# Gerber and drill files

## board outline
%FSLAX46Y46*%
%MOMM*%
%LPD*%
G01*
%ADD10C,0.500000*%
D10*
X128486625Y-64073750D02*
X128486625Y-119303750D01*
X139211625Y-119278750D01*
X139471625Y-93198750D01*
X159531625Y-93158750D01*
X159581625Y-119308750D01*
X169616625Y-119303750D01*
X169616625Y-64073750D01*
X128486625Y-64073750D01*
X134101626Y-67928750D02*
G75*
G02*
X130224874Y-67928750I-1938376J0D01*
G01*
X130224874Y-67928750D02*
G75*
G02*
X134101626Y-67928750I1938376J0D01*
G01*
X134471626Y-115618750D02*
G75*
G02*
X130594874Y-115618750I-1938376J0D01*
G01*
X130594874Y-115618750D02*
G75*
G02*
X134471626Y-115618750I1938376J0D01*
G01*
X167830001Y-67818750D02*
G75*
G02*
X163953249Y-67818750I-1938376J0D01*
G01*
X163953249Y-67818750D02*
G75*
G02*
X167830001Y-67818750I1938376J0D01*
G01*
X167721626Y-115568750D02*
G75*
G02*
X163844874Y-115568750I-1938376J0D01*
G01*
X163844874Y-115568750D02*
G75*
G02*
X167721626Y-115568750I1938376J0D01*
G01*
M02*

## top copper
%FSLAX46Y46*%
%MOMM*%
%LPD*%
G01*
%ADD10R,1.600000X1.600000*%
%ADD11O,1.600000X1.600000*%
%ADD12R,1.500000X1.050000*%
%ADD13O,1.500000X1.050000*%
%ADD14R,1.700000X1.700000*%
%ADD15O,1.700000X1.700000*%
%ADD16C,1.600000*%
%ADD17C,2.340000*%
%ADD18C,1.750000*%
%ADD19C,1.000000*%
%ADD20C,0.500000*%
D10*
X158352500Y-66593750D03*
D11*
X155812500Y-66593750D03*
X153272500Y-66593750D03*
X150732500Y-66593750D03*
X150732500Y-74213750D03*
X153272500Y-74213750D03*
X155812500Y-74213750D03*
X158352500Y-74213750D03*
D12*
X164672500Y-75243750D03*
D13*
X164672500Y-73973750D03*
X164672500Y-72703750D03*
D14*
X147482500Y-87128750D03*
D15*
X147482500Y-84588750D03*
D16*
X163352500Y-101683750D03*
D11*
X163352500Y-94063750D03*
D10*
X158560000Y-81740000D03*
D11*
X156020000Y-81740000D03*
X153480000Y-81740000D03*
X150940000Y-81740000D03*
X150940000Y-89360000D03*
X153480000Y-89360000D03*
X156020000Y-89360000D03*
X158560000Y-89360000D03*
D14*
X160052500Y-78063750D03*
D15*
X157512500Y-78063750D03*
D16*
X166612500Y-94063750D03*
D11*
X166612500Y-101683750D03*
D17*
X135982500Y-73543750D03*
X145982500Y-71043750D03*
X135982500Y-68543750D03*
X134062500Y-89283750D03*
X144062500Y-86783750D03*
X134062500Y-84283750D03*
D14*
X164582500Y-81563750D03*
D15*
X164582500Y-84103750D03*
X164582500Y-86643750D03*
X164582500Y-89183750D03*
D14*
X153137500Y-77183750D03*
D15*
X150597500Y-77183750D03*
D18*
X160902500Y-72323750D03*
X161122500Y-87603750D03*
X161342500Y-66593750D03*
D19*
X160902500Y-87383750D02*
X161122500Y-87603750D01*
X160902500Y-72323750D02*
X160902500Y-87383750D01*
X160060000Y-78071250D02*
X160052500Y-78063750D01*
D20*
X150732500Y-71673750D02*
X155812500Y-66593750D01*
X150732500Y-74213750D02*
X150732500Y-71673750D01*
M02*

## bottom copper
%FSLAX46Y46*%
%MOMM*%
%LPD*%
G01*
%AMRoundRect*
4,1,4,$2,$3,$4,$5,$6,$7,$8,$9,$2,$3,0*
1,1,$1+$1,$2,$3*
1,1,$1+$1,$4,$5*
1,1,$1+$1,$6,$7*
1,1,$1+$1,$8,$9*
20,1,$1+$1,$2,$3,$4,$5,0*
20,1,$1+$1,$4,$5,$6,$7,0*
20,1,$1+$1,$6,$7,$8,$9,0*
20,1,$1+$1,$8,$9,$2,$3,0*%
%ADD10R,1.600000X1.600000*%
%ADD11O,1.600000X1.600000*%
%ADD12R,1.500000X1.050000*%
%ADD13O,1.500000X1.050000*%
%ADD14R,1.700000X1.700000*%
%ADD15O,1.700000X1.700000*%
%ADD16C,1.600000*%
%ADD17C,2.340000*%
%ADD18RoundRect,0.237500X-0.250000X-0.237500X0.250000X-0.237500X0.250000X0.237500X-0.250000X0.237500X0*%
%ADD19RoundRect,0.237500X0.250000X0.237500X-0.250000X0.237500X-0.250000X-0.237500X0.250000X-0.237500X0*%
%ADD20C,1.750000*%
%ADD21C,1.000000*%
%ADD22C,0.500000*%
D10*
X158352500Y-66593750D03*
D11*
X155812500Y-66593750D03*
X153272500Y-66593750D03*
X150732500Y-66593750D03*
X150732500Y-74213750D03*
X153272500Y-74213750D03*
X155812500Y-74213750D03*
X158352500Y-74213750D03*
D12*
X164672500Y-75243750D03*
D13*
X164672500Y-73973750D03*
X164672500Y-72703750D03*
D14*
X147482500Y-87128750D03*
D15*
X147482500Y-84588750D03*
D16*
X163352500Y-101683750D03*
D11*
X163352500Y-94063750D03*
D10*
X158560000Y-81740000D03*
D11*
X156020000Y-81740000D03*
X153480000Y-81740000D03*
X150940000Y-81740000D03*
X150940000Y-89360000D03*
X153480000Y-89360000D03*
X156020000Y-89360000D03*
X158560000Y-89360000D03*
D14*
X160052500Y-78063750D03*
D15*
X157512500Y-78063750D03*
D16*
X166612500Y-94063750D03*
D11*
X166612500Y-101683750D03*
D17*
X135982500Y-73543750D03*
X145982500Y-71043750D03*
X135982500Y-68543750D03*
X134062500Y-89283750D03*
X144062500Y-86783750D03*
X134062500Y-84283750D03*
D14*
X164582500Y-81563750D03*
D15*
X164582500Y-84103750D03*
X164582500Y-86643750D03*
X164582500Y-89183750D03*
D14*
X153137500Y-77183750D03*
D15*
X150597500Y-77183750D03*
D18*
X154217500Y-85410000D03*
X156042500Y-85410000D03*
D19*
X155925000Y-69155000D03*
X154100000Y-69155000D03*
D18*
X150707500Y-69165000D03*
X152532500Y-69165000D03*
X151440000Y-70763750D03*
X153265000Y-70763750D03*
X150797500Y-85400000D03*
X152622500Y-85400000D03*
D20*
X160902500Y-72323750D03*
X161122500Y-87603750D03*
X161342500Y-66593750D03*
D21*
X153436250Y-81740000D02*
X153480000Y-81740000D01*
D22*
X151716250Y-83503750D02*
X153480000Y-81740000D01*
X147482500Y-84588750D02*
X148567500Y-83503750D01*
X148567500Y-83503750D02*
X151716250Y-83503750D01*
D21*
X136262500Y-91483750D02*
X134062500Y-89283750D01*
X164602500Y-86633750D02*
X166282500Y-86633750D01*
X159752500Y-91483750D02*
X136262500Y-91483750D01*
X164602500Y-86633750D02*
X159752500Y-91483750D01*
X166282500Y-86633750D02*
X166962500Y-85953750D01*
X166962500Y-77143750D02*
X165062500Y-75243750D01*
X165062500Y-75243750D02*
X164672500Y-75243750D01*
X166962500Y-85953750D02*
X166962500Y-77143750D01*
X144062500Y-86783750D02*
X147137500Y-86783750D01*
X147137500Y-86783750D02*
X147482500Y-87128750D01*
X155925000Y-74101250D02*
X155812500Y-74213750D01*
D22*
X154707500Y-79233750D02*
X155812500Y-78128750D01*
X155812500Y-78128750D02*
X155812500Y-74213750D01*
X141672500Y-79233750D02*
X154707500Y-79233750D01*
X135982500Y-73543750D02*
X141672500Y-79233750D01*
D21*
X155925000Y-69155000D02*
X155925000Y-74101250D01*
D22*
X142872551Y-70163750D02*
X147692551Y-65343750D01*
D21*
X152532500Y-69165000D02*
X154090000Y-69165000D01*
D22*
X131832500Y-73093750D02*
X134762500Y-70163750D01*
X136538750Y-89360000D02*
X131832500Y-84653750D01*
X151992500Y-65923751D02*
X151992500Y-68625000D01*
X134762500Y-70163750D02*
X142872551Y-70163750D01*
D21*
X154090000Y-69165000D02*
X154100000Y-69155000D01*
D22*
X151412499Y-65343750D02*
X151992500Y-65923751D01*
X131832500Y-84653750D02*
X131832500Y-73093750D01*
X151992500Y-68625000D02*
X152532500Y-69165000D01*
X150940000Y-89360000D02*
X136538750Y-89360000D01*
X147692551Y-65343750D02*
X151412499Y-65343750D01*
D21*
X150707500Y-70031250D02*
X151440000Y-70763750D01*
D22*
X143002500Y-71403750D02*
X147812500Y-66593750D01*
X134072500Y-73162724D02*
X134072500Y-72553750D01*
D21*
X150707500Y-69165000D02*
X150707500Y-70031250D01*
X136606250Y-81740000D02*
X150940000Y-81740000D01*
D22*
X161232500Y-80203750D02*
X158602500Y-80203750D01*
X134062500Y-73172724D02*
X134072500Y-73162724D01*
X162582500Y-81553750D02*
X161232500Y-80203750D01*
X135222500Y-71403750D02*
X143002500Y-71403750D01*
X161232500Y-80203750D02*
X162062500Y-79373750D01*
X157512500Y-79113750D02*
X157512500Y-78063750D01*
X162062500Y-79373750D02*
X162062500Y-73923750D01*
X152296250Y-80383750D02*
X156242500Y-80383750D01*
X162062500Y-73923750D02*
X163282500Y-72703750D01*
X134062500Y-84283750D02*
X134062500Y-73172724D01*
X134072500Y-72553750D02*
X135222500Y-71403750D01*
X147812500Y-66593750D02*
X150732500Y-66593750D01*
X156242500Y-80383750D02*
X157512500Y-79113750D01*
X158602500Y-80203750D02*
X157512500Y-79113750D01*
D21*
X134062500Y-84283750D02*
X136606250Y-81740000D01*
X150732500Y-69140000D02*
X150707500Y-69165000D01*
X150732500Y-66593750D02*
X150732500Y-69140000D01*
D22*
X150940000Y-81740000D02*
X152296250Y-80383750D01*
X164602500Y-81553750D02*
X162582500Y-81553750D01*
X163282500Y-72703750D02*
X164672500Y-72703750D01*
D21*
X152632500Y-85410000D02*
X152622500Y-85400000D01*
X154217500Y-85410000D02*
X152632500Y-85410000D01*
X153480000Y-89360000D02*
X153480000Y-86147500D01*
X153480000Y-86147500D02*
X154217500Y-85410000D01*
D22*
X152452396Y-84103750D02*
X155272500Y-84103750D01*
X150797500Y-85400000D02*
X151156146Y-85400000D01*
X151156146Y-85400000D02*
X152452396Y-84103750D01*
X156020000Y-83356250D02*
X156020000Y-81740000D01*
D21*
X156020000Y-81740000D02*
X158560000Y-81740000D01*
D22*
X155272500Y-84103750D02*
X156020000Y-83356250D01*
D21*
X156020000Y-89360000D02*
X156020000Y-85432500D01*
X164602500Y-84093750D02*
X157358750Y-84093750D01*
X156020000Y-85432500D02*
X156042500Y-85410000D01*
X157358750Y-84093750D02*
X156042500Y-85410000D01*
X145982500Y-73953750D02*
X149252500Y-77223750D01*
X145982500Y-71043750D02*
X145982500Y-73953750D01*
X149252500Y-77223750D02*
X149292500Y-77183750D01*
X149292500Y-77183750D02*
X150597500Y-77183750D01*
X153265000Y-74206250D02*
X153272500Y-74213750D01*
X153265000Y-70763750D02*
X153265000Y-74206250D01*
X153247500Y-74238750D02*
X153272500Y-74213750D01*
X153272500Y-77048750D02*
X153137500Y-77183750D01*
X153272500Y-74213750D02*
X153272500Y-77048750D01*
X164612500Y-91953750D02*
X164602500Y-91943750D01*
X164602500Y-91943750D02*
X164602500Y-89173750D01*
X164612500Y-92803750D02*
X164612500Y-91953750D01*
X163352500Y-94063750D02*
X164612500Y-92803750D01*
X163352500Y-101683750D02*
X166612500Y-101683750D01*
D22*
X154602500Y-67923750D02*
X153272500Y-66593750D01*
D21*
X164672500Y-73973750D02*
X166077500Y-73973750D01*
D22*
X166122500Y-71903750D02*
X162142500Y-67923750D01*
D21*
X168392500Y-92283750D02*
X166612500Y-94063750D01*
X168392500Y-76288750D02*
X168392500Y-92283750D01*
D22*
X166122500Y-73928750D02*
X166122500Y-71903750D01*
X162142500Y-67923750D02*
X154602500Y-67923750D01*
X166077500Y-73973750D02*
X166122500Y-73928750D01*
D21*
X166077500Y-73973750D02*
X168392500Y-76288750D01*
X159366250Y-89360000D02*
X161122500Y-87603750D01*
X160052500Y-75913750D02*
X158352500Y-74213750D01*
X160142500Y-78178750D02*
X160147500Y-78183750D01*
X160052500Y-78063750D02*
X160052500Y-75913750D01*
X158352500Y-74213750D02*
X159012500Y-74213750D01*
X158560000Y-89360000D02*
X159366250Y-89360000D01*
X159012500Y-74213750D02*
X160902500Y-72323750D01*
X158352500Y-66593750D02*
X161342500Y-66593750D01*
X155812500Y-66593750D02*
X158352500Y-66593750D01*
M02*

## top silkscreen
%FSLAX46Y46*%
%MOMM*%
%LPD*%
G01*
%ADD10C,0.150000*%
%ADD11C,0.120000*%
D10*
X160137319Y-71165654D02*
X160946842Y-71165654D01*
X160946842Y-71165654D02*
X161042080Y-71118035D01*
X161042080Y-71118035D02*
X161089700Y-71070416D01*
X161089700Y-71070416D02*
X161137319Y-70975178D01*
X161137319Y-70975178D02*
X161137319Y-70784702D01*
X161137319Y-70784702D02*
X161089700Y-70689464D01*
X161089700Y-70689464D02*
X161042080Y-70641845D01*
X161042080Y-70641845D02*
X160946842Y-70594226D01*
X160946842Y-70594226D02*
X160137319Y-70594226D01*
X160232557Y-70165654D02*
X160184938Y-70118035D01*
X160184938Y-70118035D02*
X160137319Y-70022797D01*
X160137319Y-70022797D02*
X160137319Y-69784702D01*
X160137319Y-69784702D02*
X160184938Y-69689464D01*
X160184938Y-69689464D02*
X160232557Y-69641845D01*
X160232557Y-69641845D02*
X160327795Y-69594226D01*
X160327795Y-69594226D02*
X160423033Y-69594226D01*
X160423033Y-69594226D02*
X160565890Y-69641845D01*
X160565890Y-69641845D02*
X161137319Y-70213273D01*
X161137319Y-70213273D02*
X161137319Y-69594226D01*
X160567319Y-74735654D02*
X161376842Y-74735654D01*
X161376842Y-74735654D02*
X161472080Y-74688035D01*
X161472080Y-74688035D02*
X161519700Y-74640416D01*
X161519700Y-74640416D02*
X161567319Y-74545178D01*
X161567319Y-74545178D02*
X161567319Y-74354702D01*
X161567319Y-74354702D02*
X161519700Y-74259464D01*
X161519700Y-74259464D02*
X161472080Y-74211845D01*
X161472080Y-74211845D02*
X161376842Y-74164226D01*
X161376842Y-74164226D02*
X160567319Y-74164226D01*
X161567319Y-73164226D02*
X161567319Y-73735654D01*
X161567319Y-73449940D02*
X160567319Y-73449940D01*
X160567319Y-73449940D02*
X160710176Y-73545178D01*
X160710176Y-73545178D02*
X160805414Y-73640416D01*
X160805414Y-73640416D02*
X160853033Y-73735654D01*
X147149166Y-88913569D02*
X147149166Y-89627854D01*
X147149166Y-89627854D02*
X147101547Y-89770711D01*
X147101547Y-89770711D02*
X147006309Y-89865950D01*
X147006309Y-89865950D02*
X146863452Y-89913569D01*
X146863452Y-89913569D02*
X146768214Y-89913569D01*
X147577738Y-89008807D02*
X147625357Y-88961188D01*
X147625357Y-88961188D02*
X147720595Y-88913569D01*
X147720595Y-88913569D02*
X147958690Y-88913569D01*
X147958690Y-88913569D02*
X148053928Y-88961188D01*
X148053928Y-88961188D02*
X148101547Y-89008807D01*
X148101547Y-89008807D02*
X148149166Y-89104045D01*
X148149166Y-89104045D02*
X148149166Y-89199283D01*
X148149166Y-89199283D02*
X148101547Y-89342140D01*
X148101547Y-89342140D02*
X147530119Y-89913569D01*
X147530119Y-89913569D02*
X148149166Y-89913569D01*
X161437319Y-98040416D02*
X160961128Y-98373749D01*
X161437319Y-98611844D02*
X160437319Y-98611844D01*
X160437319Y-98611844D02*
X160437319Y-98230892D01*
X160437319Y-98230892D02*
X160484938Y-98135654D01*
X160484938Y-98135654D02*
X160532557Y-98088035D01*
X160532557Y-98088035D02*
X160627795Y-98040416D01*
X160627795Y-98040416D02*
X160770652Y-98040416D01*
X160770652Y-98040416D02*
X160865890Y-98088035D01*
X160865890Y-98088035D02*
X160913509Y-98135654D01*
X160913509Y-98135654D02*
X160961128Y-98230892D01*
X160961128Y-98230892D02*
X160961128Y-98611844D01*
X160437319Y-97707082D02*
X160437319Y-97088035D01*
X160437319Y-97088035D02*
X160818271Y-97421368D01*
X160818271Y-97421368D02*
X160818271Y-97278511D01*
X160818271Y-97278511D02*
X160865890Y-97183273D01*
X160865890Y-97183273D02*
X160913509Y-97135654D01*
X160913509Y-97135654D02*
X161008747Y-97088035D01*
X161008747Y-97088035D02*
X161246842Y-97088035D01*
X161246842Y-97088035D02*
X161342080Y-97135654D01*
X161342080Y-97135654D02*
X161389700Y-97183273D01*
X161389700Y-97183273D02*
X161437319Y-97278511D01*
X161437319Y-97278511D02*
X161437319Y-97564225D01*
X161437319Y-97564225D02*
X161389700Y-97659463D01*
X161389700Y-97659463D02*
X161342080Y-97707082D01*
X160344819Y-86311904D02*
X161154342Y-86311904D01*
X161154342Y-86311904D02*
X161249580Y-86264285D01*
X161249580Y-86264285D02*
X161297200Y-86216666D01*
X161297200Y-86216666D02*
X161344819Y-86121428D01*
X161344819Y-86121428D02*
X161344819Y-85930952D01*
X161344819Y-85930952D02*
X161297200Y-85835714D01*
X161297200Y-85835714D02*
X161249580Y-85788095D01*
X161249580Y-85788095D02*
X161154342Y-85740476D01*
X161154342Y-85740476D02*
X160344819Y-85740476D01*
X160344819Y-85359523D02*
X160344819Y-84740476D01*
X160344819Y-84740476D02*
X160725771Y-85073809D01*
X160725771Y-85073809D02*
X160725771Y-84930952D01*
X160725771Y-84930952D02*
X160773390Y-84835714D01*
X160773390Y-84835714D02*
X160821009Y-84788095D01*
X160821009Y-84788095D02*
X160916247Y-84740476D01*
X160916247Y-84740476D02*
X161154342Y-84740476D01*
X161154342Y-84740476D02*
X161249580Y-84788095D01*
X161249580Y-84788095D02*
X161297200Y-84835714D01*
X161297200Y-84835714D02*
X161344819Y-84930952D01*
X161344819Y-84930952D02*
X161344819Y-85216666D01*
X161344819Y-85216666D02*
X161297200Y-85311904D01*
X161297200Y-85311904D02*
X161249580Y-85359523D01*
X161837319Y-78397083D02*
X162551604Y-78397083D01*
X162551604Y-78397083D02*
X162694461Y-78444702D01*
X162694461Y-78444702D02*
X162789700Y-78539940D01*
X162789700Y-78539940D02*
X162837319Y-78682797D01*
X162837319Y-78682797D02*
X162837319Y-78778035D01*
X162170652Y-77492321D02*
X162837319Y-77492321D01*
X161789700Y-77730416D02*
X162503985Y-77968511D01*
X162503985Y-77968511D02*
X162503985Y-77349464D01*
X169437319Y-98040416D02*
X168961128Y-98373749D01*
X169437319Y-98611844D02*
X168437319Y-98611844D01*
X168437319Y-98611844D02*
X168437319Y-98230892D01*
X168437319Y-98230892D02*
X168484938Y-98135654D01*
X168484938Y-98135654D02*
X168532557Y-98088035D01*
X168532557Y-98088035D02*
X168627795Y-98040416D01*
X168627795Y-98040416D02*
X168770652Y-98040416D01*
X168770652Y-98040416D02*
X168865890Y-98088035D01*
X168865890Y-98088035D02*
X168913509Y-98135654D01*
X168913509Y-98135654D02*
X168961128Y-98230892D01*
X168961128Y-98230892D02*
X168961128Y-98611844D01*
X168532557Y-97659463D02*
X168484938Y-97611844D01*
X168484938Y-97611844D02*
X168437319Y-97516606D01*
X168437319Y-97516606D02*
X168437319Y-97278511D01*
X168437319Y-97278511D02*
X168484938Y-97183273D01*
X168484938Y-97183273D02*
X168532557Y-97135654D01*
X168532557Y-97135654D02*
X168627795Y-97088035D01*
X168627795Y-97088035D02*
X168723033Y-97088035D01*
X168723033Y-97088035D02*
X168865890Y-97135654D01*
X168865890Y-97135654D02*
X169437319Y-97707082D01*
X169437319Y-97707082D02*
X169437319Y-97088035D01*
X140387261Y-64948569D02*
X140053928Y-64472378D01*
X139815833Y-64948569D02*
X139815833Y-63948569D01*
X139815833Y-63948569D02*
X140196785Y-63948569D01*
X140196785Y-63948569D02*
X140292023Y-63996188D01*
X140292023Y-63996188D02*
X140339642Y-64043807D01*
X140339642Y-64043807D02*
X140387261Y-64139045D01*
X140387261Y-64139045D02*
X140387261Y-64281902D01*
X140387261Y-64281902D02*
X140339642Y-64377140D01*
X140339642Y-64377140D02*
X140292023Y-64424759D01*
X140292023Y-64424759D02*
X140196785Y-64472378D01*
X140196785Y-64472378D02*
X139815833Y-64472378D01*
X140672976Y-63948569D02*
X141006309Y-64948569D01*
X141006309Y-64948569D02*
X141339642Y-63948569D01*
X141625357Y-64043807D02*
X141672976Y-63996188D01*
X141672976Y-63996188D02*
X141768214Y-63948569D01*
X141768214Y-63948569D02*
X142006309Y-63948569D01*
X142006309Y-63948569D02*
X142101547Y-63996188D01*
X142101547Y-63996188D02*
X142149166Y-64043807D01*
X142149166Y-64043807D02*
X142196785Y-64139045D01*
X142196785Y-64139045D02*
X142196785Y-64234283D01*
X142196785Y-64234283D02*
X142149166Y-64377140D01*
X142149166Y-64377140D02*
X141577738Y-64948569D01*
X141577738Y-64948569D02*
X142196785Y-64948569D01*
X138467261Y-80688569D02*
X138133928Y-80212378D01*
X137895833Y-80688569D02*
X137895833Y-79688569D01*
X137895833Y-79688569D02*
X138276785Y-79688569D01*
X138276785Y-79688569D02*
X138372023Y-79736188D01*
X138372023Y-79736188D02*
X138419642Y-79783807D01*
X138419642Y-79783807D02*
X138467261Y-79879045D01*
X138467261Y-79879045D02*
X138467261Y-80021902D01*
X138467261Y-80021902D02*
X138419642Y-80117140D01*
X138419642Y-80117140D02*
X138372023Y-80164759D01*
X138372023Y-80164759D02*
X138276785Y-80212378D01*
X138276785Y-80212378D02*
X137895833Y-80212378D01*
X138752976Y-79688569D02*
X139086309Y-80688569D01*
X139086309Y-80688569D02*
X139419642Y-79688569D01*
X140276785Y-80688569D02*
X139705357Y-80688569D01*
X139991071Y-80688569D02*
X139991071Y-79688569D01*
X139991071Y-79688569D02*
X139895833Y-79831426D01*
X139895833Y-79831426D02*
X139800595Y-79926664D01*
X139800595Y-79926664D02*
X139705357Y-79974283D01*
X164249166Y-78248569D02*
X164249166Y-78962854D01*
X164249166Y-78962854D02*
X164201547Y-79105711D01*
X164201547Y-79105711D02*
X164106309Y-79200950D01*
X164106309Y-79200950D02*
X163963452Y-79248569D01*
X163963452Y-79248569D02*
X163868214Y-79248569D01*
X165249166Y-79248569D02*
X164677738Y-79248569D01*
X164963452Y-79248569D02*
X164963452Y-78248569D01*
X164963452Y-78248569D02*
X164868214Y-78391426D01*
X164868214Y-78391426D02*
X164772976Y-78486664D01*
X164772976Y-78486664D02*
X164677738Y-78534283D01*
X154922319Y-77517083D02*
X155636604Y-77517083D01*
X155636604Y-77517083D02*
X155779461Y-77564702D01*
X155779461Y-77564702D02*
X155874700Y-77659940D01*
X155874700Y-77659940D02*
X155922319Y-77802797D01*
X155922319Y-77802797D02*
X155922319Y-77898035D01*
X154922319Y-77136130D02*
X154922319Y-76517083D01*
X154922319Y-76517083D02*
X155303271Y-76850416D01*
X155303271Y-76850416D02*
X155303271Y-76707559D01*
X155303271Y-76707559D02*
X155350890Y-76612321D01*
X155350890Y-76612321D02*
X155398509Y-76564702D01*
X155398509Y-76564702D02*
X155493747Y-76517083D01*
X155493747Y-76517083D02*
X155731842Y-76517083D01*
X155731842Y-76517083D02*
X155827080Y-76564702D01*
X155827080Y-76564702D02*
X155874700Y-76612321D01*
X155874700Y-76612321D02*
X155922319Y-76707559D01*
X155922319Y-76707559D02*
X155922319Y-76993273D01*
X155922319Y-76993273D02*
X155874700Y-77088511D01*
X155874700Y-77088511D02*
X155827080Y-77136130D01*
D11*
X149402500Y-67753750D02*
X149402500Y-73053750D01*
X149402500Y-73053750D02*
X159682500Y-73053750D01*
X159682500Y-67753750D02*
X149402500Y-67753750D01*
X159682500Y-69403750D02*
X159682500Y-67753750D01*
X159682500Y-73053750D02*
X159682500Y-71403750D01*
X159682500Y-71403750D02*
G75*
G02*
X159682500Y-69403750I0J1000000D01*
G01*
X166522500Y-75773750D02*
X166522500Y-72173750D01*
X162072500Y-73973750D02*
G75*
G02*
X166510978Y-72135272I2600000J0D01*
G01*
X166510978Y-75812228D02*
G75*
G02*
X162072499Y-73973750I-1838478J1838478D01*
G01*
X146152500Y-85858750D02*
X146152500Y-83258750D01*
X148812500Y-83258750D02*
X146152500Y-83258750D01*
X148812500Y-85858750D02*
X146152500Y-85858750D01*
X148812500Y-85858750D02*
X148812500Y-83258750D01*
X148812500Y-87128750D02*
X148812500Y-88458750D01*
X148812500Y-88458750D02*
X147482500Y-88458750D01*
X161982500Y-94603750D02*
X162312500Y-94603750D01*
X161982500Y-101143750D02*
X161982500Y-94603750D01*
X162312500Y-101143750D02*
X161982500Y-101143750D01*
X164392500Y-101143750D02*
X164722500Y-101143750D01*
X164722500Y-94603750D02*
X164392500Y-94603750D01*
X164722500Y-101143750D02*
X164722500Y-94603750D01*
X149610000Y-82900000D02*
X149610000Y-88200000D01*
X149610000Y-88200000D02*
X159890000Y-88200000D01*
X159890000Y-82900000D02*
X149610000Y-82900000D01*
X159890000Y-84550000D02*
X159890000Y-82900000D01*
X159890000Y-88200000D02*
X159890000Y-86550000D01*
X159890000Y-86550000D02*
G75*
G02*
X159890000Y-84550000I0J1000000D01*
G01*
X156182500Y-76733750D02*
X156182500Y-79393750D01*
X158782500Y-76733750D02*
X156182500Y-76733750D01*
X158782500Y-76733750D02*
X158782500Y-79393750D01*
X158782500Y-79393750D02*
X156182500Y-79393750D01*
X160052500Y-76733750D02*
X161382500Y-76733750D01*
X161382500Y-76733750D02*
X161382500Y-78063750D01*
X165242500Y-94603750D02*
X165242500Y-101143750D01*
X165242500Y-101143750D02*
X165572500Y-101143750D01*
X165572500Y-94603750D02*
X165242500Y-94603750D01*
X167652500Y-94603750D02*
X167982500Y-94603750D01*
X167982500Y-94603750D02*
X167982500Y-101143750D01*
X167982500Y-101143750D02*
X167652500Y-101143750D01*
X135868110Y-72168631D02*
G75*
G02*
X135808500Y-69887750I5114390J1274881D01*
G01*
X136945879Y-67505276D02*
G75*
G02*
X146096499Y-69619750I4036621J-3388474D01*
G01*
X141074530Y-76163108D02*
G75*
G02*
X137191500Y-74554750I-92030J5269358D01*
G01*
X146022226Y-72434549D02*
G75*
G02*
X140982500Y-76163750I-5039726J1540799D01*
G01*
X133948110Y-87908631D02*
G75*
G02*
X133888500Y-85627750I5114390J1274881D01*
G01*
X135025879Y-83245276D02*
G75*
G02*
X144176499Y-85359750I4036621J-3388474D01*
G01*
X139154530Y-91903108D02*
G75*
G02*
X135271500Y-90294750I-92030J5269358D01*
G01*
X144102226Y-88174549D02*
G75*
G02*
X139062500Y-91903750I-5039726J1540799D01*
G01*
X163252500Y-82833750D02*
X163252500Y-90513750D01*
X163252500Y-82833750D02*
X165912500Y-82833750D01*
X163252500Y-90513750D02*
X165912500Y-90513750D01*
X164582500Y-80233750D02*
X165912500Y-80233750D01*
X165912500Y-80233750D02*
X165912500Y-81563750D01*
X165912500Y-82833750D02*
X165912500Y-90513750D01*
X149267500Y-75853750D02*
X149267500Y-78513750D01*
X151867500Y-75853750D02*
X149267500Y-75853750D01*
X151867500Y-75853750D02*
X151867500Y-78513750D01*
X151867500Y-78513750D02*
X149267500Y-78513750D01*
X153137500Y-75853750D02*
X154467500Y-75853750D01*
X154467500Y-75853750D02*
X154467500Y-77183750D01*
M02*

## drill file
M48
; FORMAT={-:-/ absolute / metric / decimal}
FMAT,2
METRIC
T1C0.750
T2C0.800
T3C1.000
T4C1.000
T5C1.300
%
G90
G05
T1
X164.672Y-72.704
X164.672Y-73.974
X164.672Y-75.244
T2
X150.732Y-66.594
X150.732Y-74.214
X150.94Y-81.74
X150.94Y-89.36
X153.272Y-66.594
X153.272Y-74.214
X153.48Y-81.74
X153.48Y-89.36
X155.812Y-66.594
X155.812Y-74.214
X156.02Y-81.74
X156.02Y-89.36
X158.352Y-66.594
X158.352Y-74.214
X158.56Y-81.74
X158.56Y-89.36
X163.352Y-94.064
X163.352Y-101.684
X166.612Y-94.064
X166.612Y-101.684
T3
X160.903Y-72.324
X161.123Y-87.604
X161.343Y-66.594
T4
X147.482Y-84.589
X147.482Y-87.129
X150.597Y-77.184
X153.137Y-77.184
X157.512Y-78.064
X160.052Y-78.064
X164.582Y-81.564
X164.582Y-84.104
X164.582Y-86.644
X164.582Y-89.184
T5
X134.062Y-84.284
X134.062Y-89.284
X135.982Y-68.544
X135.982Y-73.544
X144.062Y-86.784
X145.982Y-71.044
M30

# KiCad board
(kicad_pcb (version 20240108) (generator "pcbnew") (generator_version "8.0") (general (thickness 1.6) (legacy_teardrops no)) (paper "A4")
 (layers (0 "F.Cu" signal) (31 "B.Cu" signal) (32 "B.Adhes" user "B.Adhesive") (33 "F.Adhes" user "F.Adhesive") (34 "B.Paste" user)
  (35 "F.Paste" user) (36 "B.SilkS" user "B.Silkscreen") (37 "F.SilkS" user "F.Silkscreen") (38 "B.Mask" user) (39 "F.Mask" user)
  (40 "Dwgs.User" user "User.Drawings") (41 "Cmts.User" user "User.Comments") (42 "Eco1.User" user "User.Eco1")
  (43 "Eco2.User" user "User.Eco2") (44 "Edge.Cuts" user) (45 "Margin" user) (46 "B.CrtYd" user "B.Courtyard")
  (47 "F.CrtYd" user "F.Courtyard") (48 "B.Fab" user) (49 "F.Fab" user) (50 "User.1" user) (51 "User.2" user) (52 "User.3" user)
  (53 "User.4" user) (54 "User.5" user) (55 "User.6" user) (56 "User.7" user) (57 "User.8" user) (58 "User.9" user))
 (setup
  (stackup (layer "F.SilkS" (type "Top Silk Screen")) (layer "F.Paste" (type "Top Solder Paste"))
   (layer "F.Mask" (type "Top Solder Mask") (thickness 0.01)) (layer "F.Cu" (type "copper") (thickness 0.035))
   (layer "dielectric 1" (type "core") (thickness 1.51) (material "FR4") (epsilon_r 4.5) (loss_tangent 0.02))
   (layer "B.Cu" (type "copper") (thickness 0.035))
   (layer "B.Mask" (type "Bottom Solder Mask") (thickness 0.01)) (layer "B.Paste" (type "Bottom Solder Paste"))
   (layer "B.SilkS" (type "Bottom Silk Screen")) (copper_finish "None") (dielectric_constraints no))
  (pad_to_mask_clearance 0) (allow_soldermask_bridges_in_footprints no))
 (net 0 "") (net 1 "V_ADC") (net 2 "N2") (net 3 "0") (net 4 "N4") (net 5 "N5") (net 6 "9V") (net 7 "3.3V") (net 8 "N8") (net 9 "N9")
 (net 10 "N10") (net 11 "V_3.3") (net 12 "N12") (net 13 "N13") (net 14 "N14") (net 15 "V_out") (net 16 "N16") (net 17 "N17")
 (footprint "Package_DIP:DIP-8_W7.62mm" (layer "F.Cu") (at 158.3525 66.59375 -90)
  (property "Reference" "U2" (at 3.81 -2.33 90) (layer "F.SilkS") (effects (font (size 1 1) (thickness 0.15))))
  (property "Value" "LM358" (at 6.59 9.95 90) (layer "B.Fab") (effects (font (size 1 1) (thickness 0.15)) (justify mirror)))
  (fp_line (start 1.16 8.95) (end 6.46 8.95) (stroke (width 0.12) (type solid)) (layer "F.SilkS"))
  (fp_line (start 6.46 8.95) (end 6.46 -1.33) (stroke (width 0.12) (type solid)) (layer "F.SilkS"))
  (fp_line (start 1.16 -1.33) (end 1.16 8.95) (stroke (width 0.12) (type solid)) (layer "F.SilkS"))
  (fp_line (start 2.81 -1.33) (end 1.16 -1.33) (stroke (width 0.12) (type solid)) (layer "F.SilkS"))
  (fp_line (start 6.46 -1.33) (end 4.81 -1.33) (stroke (width 0.12) (type solid)) (layer "F.SilkS"))
  (fp_arc (start 4.81 -1.33) (mid 3.81 -0.33) (end 2.81 -1.33) (stroke (width 0.12) (type solid)) (layer "F.SilkS"))
  (pad "1" thru_hole rect (at 0 0 270) (size 1.6 1.6) (drill 0.8) (layers "*.Cu" "*.Mask") (remove_unused_layers no) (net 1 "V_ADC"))
  (pad "2" thru_hole oval (at 0 2.54 270) (size 1.6 1.6) (drill 0.8) (layers "*.Cu" "*.Mask") (remove_unused_layers no) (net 1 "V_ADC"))
  (pad "3" thru_hole oval (at 0 5.08 270) (size 1.6 1.6) (drill 0.8) (layers "*.Cu" "*.Mask") (remove_unused_layers no) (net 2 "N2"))
  (pad "4" thru_hole oval (at 0 7.62 270) (size 1.6 1.6) (drill 0.8) (layers "*.Cu" "*.Mask") (remove_unused_layers no) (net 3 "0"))
  (pad "5" thru_hole oval (at 7.62 7.62 270) (size 1.6 1.6) (drill 0.8) (layers "*.Cu" "*.Mask") (remove_unused_layers no) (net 1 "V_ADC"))
  (pad "6" thru_hole oval (at 7.62 5.08 270) (size 1.6 1.6) (drill 0.8) (layers "*.Cu" "*.Mask") (remove_unused_layers no) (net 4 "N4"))
  (pad "7" thru_hole oval (at 7.62 2.54 270) (size 1.6 1.6) (drill 0.8) (layers "*.Cu" "*.Mask") (remove_unused_layers no) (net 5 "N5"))
  (pad "8" thru_hole oval (at 7.62 0 270) (size 1.6 1.6) (drill 0.8) (layers "*.Cu" "*.Mask") (remove_unused_layers no) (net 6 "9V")))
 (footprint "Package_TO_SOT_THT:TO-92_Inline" (layer "F.Cu") (at 164.6725 75.24375 90)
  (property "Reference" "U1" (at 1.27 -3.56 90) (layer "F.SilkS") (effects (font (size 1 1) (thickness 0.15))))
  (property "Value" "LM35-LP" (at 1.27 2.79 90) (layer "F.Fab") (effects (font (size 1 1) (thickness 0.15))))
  (fp_line (start -0.53 1.85) (end 3.07 1.85) (stroke (width 0.12) (type solid)) (layer "F.SilkS"))
  (fp_arc (start 1.27 -2.6) (mid 3.672087 -0.994977) (end 3.108478 1.838478) (stroke (width 0.12) (type solid)) (layer "F.SilkS"))
  (fp_arc (start -0.568478 1.838478) (mid -1.132087 -0.994977) (end 1.27 -2.6) (stroke (width 0.12) (type solid)) (layer "F.SilkS"))
  (pad "1" thru_hole rect (at 0 0 90) (size 1.05 1.5) (drill 0.75) (layers "*.Cu" "*.Mask") (remove_unused_layers no) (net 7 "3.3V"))
  (pad "2" thru_hole oval (at 1.27 0 90) (size 1.05 1.5) (drill 0.75) (layers "*.Cu" "*.Mask") (remove_unused_layers no) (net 2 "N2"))
  (pad "3" thru_hole oval (at 2.54 0 90) (size 1.05 1.5) (drill 0.75) (layers "*.Cu" "*.Mask") (remove_unused_layers no) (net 3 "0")))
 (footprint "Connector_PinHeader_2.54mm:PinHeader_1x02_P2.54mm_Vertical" (layer "F.Cu") (at 147.4825 87.12875 180)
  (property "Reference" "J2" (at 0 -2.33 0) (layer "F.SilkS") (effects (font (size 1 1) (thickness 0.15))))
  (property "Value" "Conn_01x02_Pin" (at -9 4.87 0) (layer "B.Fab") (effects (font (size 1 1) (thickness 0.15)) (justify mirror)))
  (fp_line (start 1.33 1.27) (end 1.33 3.87) (stroke (width 0.12) (type solid)) (layer "F.SilkS"))
  (fp_line (start -1.33 3.87) (end 1.33 3.87) (stroke (width 0.12) (type solid)) (layer "F.SilkS"))
  (fp_line (start -1.33 1.27) (end 1.33 1.27) (stroke (width 0.12) (type solid)) (layer "F.SilkS"))
  (fp_line (start -1.33 1.27) (end -1.33 3.87) (stroke (width 0.12) (type solid)) (layer "F.SilkS"))
  (fp_line (start -1.33 0) (end -1.33 -1.33) (stroke (width 0.12) (type solid)) (layer "F.SilkS"))
  (fp_line (start -1.33 -1.33) (end 0 -1.33) (stroke (width 0.12) (type solid)) (layer "F.SilkS"))
  (pad "1" thru_hole rect (at 0 0 180) (size 1.7 1.7) (drill 1) (layers "*.Cu" "*.Mask") (remove_unused_layers no) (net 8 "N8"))
  (pad "2" thru_hole oval (at 0 2.54 180) (size 1.7 1.7) (drill 1) (layers "*.Cu" "*.Mask") (remove_unused_layers no) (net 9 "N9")))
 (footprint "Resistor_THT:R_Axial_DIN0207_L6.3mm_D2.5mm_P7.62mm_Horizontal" (layer "F.Cu") (at 163.3525 101.68375 90)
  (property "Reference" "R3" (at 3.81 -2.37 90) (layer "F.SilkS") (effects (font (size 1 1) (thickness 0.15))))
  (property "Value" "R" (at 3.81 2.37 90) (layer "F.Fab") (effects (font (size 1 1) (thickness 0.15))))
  (fp_line (start 7.08 -1.37) (end 7.08 -1.04) (stroke (width 0.12) (type solid)) (layer "F.SilkS"))
  (fp_line (start 0.54 -1.37) (end 7.08 -1.37) (stroke (width 0.12) (type solid)) (layer "F.SilkS"))
  (fp_line (start 0.54 -1.04) (end 0.54 -1.37) (stroke (width 0.12) (type solid)) (layer "F.SilkS"))
  (fp_line (start 0.54 1.04) (end 0.54 1.37) (stroke (width 0.12) (type solid)) (layer "F.SilkS"))
  (fp_line (start 7.08 1.37) (end 7.08 1.04) (stroke (width 0.12) (type solid)) (layer "F.SilkS"))
  (fp_line (start 0.54 1.37) (end 7.08 1.37) (stroke (width 0.12) (type solid)) (layer "F.SilkS"))
  (pad "1" thru_hole circle (at 0 0 90) (size 1.6 1.6) (drill 0.8) (layers "*.Cu" "*.Mask") (remove_unused_layers no) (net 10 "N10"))
  (pad "2" thru_hole oval (at 7.62 0 90) (size 1.6 1.6) (drill 0.8) (layers "*.Cu" "*.Mask") (remove_unused_layers no) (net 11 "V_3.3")))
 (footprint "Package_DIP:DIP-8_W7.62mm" (layer "F.Cu") (at 158.56 81.74 -90)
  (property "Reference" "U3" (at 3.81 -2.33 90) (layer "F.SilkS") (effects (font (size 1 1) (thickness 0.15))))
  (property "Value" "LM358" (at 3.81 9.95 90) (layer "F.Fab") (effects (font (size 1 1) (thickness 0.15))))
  (fp_line (start 1.16 8.95) (end 6.46 8.95) (stroke (width 0.12) (type solid)) (layer "F.SilkS"))
  (fp_line (start 6.46 8.95) (end 6.46 -1.33) (stroke (width 0.12) (type solid)) (layer "F.SilkS"))
  (fp_line (start 1.16 -1.33) (end 1.16 8.95) (stroke (width 0.12) (type solid)) (layer "F.SilkS"))
  (fp_line (start 2.81 -1.33) (end 1.16 -1.33) (stroke (width 0.12) (type solid)) (layer "F.SilkS"))
  (fp_line (start 6.46 -1.33) (end 4.81 -1.33) (stroke (width 0.12) (type solid)) (layer "F.SilkS"))
  (fp_arc (start 4.81 -1.33) (mid 3.81 -0.33) (end 2.81 -1.33) (stroke (width 0.12) (type solid)) (layer "F.SilkS"))
  (pad "1" thru_hole rect (at 0 0 270) (size 1.6 1.6) (drill 0.8) (layers "*.Cu" "*.Mask") (remove_unused_layers no) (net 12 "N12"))
  (pad "2" thru_hole oval (at 0 2.54 270) (size 1.6 1.6) (drill 0.8) (layers "*.Cu" "*.Mask") (remove_unused_layers no) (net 12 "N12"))
  (pad "3" thru_hole oval (at 0 5.08 270) (size 1.6 1.6) (drill 0.8) (layers "*.Cu" "*.Mask") (remove_unused_layers no) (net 9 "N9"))
  (pad "4" thru_hole oval (at 0 7.62 270) (size 1.6 1.6) (drill 0.8) (layers "*.Cu" "*.Mask") (remove_unused_layers no) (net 3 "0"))
  (pad "5" thru_hole oval (at 7.62 7.62 270) (size 1.6 1.6) (drill 0.8) (layers "*.Cu" "*.Mask") (remove_unused_layers no) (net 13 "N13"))
  (pad "6" thru_hole oval (at 7.62 5.08 270) (size 1.6 1.6) (drill 0.8) (layers "*.Cu" "*.Mask") (remove_unused_layers no) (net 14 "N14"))
  (pad "7" thru_hole oval (at 7.62 2.54 270) (size 1.6 1.6) (drill 0.8) (layers "*.Cu" "*.Mask") (remove_unused_layers no) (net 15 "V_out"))
  (pad "8" thru_hole oval (at 7.62 0 270) (size 1.6 1.6) (drill 0.8) (layers "*.Cu" "*.Mask") (remove_unused_layers no) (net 6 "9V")))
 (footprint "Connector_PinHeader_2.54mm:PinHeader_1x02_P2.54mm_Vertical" (layer "F.Cu") (at 160.0525 78.06375 -90)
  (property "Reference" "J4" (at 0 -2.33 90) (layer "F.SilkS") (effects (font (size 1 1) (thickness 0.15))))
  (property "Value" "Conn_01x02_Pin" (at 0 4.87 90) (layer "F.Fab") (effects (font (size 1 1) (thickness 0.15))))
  (fp_line (start -1.33 3.87) (end 1.33 3.87) (stroke (width 0.12) (type solid)) (layer "F.SilkS"))
  (fp_line (start -1.33 1.27) (end -1.33 3.87) (stroke (width 0.12) (type solid)) (layer "F.SilkS"))
  (fp_line (start -1.33 1.27) (end 1.33 1.27) (stroke (width 0.12) (type solid)) (layer "F.SilkS"))
  (fp_line (start 1.33 1.27) (end 1.33 3.87) (stroke (width 0.12) (type solid)) (layer "F.SilkS"))
  (fp_line (start -1.33 0) (end -1.33 -1.33) (stroke (width 0.12) (type solid)) (layer "F.SilkS"))
  (fp_line (start -1.33 -1.33) (end 0 -1.33) (stroke (width 0.12) (type solid)) (layer "F.SilkS"))
  (pad "1" thru_hole rect (at 0 0 270) (size 1.7 1.7) (drill 1) (layers "*.Cu" "*.Mask") (remove_unused_layers no) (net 6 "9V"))
  (pad "2" thru_hole oval (at 0 2.54 270) (size 1.7 1.7) (drill 1) (layers "*.Cu" "*.Mask") (remove_unused_layers no) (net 3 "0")))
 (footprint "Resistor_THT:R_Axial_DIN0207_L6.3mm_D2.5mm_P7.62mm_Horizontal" (layer "F.Cu") (at 166.6125 94.06375 -90)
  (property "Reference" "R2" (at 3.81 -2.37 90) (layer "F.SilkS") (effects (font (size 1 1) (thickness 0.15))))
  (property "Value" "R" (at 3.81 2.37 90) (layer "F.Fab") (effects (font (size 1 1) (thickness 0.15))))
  (fp_line (start 0.54 1.37) (end 7.08 1.37) (stroke (width 0.12) (type solid)) (layer "F.SilkS"))
  (fp_line (start 7.08 1.37) (end 7.08 1.04) (stroke (width 0.12) (type solid)) (layer "F.SilkS"))
  (fp_line (start 0.54 1.04) (end 0.54 1.37) (stroke (width 0.12) (type solid)) (layer "F.SilkS"))
  (fp_line (start 0.54 -1.04) (end 0.54 -1.37) (stroke (width 0.12) (type solid)) (layer "F.SilkS"))
  (fp_line (start 0.54 -1.37) (end 7.08 -1.37) (stroke (width 0.12) (type solid)) (layer "F.SilkS"))
  (fp_line (start 7.08 -1.37) (end 7.08 -1.04) (stroke (width 0.12) (type solid)) (layer "F.SilkS"))
  (pad "1" thru_hole circle (at 0 0 270) (size 1.6 1.6) (drill 0.8) (layers "*.Cu" "*.Mask") (remove_unused_layers no) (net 2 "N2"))
  (pad "2" thru_hole oval (at 7.62 0 270) (size 1.6 1.6) (drill 0.8) (layers "*.Cu" "*.Mask") (remove_unused_layers no) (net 10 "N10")))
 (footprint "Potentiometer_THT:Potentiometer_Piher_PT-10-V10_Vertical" (layer "F.Cu") (at 135.9825 73.54375)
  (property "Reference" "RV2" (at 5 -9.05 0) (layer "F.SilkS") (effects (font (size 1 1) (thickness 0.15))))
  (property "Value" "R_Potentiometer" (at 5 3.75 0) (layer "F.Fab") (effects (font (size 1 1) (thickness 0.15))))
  (fp_arc (start -0.11439 -1.375119) (mid -0.269093 -2.512295) (end -0.174 -3.656) (stroke (width 0.12) (type solid)) (layer "F.SilkS"))
  (fp_arc (start 0.963379 -6.038474) (mid 6.186565 -7.784991) (end 10.114 -3.924) (stroke (width 0.12) (type solid)) (layer "F.SilkS"))
  (fp_arc (start 5.09203 2.619358) (mid 2.983245 2.219015) (end 1.209 1.011) (stroke (width 0.12) (type solid)) (layer "F.SilkS"))
  (fp_arc (start 10.039726 -1.109201) (mid 8.134716 1.586326) (end 5 2.62) (stroke (width 0.12) (type solid)) (layer "F.SilkS"))
  (pad "1" thru_hole circle (at 0 0) (size 2.34 2.34) (drill 1.3) (layers "*.Cu" "*.Mask") (remove_unused_layers no) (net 5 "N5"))
  (pad "2" thru_hole circle (at 10 -2.5) (size 2.34 2.34) (drill 1.3) (layers "*.Cu" "*.Mask") (remove_unused_layers no) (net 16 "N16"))
  (pad "3" thru_hole circle (at 0 -5) (size 2.34 2.34) (drill 1.3) (layers "*.Cu" "*.Mask") (remove_unused_layers no) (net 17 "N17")))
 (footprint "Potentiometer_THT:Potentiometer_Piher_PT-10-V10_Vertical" (layer "F.Cu") (at 134.0625 89.28375)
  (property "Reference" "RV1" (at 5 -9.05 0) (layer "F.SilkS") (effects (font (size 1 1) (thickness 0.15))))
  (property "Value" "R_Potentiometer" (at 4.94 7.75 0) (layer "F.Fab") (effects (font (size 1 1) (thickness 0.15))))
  (fp_arc (start -0.11439 -1.375119) (mid -0.269093 -2.512295) (end -0.174 -3.656) (stroke (width 0.12) (type solid)) (layer "F.SilkS"))
  (fp_arc (start 0.963379 -6.038474) (mid 6.186565 -7.784991) (end 10.114 -3.924) (stroke (width 0.12) (type solid)) (layer "F.SilkS"))
  (fp_arc (start 5.09203 2.619358) (mid 2.983245 2.219015) (end 1.209 1.011) (stroke (width 0.12) (type solid)) (layer "F.SilkS"))
  (fp_arc (start 10.039726 -1.109201) (mid 8.134716 1.586326) (end 5 2.62) (stroke (width 0.12) (type solid)) (layer "F.SilkS"))
  (pad "1" thru_hole circle (at 0 0) (size 2.34 2.34) (drill 1.3) (layers "*.Cu" "*.Mask") (remove_unused_layers no) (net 7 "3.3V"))
  (pad "2" thru_hole circle (at 10 -2.5) (size 2.34 2.34) (drill 1.3) (layers "*.Cu" "*.Mask") (remove_unused_layers no) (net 8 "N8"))
  (pad "3" thru_hole circle (at 0 -5) (size 2.34 2.34) (drill 1.3) (layers "*.Cu" "*.Mask") (remove_unused_layers no) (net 3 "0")))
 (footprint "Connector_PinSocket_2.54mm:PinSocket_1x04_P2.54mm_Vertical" (layer "F.Cu") (at 164.5825 81.56375)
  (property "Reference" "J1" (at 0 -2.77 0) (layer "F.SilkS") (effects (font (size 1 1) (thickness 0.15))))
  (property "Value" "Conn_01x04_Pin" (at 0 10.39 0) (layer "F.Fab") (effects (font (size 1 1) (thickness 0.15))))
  (fp_line (start -1.33 1.27) (end -1.33 8.95) (stroke (width 0.12) (type solid)) (layer "F.SilkS"))
  (fp_line (start -1.33 1.27) (end 1.33 1.27) (stroke (width 0.12) (type solid)) (layer "F.SilkS"))
  (fp_line (start -1.33 8.95) (end 1.33 8.95) (stroke (width 0.12) (type solid)) (layer "F.SilkS"))
  (fp_line (start 0 -1.33) (end 1.33 -1.33) (stroke (width 0.12) (type solid)) (layer "F.SilkS"))
  (fp_line (start 1.33 -1.33) (end 1.33 0) (stroke (width 0.12) (type solid)) (layer "F.SilkS"))
  (fp_line (start 1.33 1.27) (end 1.33 8.95) (stroke (width 0.12) (type solid)) (layer "F.SilkS"))
  (pad "1" thru_hole rect (at 0 0) (size 1.7 1.7) (drill 1) (layers "*.Cu" "*.Mask") (remove_unused_layers no) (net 3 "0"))
  (pad "2" thru_hole oval (at 0 2.54) (size 1.7 1.7) (drill 1) (layers "*.Cu" "*.Mask") (remove_unused_layers no) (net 15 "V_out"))
  (pad "3" thru_hole oval (at 0 5.08) (size 1.7 1.7) (drill 1) (layers "*.Cu" "*.Mask") (remove_unused_layers no) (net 7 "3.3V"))
  (pad "4" thru_hole oval (at 0 7.62) (size 1.7 1.7) (drill 1) (layers "*.Cu" "*.Mask") (remove_unused_layers no) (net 11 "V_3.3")))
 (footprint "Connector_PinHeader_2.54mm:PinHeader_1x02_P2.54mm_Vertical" (layer "F.Cu") (at 153.1375 77.18375 -90)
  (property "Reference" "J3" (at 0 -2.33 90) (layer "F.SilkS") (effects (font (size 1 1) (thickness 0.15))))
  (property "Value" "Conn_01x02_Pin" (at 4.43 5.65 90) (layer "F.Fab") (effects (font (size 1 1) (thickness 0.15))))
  (fp_line (start -1.33 3.87) (end 1.33 3.87) (stroke (width 0.12) (type solid)) (layer "F.SilkS"))
  (fp_line (start -1.33 1.27) (end -1.33 3.87) (stroke (width 0.12) (type solid)) (layer "F.SilkS"))
  (fp_line (start -1.33 1.27) (end 1.33 1.27) (stroke (width 0.12) (type solid)) (layer "F.SilkS"))
  (fp_line (start 1.33 1.27) (end 1.33 3.87) (stroke (width 0.12) (type solid)) (layer "F.SilkS"))
  (fp_line (start -1.33 0) (end -1.33 -1.33) (stroke (width 0.12) (type solid)) (layer "F.SilkS"))
  (fp_line (start -1.33 -1.33) (end 0 -1.33) (stroke (width 0.12) (type solid)) (layer "F.SilkS"))
  (pad "1" thru_hole rect (at 0 0 270) (size 1.7 1.7) (drill 1) (layers "*.Cu" "*.Mask") (remove_unused_layers no) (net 4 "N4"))
  (pad "2" thru_hole oval (at 0 2.54 270) (size 1.7 1.7) (drill 1) (layers "*.Cu" "*.Mask") (remove_unused_layers no) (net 16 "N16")))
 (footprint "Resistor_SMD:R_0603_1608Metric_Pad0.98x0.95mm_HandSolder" (layer "B.Cu") (at 155.13 85.41)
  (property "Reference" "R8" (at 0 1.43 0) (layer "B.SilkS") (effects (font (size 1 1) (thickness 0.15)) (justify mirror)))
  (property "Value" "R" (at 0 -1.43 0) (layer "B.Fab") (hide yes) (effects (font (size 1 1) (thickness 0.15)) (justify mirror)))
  (pad "1" smd roundrect (at -0.9125 0) (size 0.975 0.95) (layers "B.Cu" "B.Paste" "B.Mask") (roundrect_rratio 0.25) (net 14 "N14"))
  (pad "2" smd roundrect (at 0.9125 0) (size 0.975 0.95) (layers "B.Cu" "B.Paste" "B.Mask") (roundrect_rratio 0.25) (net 15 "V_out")))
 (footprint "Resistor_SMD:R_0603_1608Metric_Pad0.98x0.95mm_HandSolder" (layer "B.Cu") (at 155.0125 69.155 180)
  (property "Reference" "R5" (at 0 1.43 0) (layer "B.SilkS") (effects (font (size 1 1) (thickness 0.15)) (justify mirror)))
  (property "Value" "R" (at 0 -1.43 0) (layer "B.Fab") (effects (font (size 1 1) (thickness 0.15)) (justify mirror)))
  (pad "1" smd roundrect (at -0.9125 0 180) (size 0.975 0.95) (layers "B.Cu" "B.Paste" "B.Mask") (roundrect_rratio 0.25) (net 5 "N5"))
  (pad "2" smd roundrect (at 0.9125 0 180) (size 0.975 0.95) (layers "B.Cu" "B.Paste" "B.Mask") (roundrect_rratio 0.25) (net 13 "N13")))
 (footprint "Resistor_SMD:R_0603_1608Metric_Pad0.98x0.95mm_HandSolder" (layer "B.Cu") (at 151.62 69.165)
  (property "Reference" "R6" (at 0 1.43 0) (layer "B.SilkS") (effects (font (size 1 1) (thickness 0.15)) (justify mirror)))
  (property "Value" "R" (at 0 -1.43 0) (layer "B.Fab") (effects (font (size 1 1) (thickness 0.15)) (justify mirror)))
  (pad "1" smd roundrect (at -0.9125 0) (size 0.975 0.95) (layers "B.Cu" "B.Paste" "B.Mask") (roundrect_rratio 0.25) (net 3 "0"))
  (pad "2" smd roundrect (at 0.9125 0) (size 0.975 0.95) (layers "B.Cu" "B.Paste" "B.Mask") (roundrect_rratio 0.25) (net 13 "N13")))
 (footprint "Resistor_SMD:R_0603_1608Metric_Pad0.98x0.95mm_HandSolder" (layer "B.Cu") (at 152.3525 70.76375)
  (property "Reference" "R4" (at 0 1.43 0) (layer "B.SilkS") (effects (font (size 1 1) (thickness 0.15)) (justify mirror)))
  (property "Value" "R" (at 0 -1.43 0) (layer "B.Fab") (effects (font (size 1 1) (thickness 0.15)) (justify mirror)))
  (pad "1" smd roundrect (at -0.9125 0) (size 0.975 0.95) (layers "B.Cu" "B.Paste" "B.Mask") (roundrect_rratio 0.25) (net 3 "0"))
  (pad "2" smd roundrect (at 0.9125 0) (size 0.975 0.95) (layers "B.Cu" "B.Paste" "B.Mask") (roundrect_rratio 0.25) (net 4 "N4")))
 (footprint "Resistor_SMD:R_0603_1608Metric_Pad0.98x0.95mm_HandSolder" (layer "B.Cu") (at 151.71 85.4)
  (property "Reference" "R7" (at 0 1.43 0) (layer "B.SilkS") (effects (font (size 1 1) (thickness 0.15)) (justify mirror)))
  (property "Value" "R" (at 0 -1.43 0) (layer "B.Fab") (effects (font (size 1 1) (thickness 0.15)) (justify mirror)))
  (pad "1" smd roundrect (at -0.9125 0) (size 0.975 0.95) (layers "B.Cu" "B.Paste" "B.Mask") (roundrect_rratio 0.25) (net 12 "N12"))
  (pad "2" smd roundrect (at 0.9125 0) (size 0.975 0.95) (layers "B.Cu" "B.Paste" "B.Mask") (roundrect_rratio 0.25) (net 14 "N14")))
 (gr_poly
  (pts (xy 128.486625 64.07375) (xy 128.486625 119.30375) (xy 139.211625 119.27875) (xy 139.471625 93.19875) (xy 159.531625 93.15875)
   (xy 159.581625 119.30875) (xy 169.616625 119.30375) (xy 169.616625 64.07375))
  (stroke (width 0.5) (type solid)) (fill none) (layer "Edge.Cuts"))
 (gr_circle (center 132.16325 67.92875) (end 134.101626 67.92875) (stroke (width 0.5) (type default)) (fill none) (layer "Edge.Cuts"))
 (gr_circle (center 132.53325 115.61875) (end 134.471626 115.61875) (stroke (width 0.5) (type default)) (fill none) (layer "Edge.Cuts"))
 (gr_circle (center 165.891625 67.81875) (end 167.830001 67.81875) (stroke (width 0.5) (type default)) (fill none) (layer "Edge.Cuts"))
 (gr_circle (center 165.78325 115.56875) (end 167.721626 115.56875) (stroke (width 0.5) (type default)) (fill none) (layer "Edge.Cuts"))
 (segment (start 153.43625 81.74) (end 153.48 81.74) (width 1) (layer "B.Cu") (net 9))
 (segment (start 151.71625 83.50375) (end 153.48 81.74) (width 0.5) (layer "B.Cu") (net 9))
 (segment (start 147.4825 84.58875) (end 148.5675 83.50375) (width 0.5) (layer "B.Cu") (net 9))
 (segment (start 148.5675 83.50375) (end 151.71625 83.50375) (width 0.5) (layer "B.Cu") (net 9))
 (segment (start 136.2625 91.48375) (end 134.0625 89.28375) (width 1) (layer "B.Cu") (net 7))
 (segment (start 164.6025 86.63375) (end 166.2825 86.63375) (width 1) (layer "B.Cu") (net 7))
 (segment (start 159.7525 91.48375) (end 136.2625 91.48375) (width 1) (layer "B.Cu") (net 7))
 (segment (start 164.6025 86.63375) (end 159.7525 91.48375) (width 1) (layer "B.Cu") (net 7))
 (segment (start 166.2825 86.63375) (end 166.9625 85.95375) (width 1) (layer "B.Cu") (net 7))
 (segment (start 166.9625 77.14375) (end 165.0625 75.24375) (width 1) (layer "B.Cu") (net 7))
 (segment (start 165.0625 75.24375) (end 164.6725 75.24375) (width 1) (layer "B.Cu") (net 7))
 (segment (start 166.9625 85.95375) (end 166.9625 77.14375) (width 1) (layer "B.Cu") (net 7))
 (segment (start 144.0625 86.78375) (end 147.1375 86.78375) (width 1) (layer "B.Cu") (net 8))
 (segment (start 147.1375 86.78375) (end 147.4825 87.12875) (width 1) (layer "B.Cu") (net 8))
 (segment (start 155.925 74.10125) (end 155.8125 74.21375) (width 1) (layer "B.Cu") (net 5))
 (segment (start 154.7075 79.23375) (end 155.8125 78.12875) (width 0.5) (layer "B.Cu") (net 5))
 (segment (start 155.8125 78.12875) (end 155.8125 74.21375) (width 0.5) (layer "B.Cu") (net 5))
 (segment (start 141.6725 79.23375) (end 154.7075 79.23375) (width 0.5) (layer "B.Cu") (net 5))
 (segment (start 135.9825 73.54375) (end 141.6725 79.23375) (width 0.5) (layer "B.Cu") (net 5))
 (segment (start 155.925 69.155) (end 155.925 74.10125) (width 1) (layer "B.Cu") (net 5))
 (segment (start 142.872551 70.16375) (end 147.692551 65.34375) (width 0.5) (layer "B.Cu") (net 13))
 (segment (start 152.5325 69.165) (end 154.09 69.165) (width 1) (layer "B.Cu") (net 13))
 (segment (start 131.8325 73.09375) (end 134.7625 70.16375) (width 0.5) (layer "B.Cu") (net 13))
 (segment (start 136.53875 89.36) (end 131.8325 84.65375) (width 0.5) (layer "B.Cu") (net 13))
 (segment (start 151.9925 65.923751) (end 151.9925 68.625) (width 0.5) (layer "B.Cu") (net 13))
 (segment (start 134.7625 70.16375) (end 142.872551 70.16375) (width 0.5) (layer "B.Cu") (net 13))
 (segment (start 154.09 69.165) (end 154.1 69.155) (width 1) (layer "B.Cu") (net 13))
 (segment (start 151.412499 65.34375) (end 151.9925 65.923751) (width 0.5) (layer "B.Cu") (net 13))
 (segment (start 131.8325 84.65375) (end 131.8325 73.09375) (width 0.5) (layer "B.Cu") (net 13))
 (segment (start 151.9925 68.625) (end 152.5325 69.165) (width 0.5) (layer "B.Cu") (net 13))
 (segment (start 150.94 89.36) (end 136.53875 89.36) (width 0.5) (layer "B.Cu") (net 13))
 (segment (start 147.692551 65.34375) (end 151.412499 65.34375) (width 0.5) (layer "B.Cu") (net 13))
 (segment (start 150.7075 70.03125) (end 151.44 70.76375) (width 1) (layer "B.Cu") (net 3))
 (segment (start 143.0025 71.40375) (end 147.8125 66.59375) (width 0.5) (layer "B.Cu") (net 3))
 (segment (start 134.0725 73.162724) (end 134.0725 72.55375) (width 0.5) (layer "B.Cu") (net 3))
 (segment (start 150.7075 69.165) (end 150.7075 70.03125) (width 1) (layer "B.Cu") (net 3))
 (segment (start 136.60625 81.74) (end 150.94 81.74) (width 1) (layer "B.Cu") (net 3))
 (segment (start 161.2325 80.20375) (end 158.6025 80.20375) (width 0.5) (layer "B.Cu") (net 3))
 (segment (start 134.0625 73.172724) (end 134.0725 73.162724) (width 0.5) (layer "B.Cu") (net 3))
 (segment (start 162.5825 81.55375) (end 161.2325 80.20375) (width 0.5) (layer "B.Cu") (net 3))
 (segment (start 135.2225 71.40375) (end 143.0025 71.40375) (width 0.5) (layer "B.Cu") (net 3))
 (segment (start 161.2325 80.20375) (end 162.0625 79.37375) (width 0.5) (layer "B.Cu") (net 3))
 (segment (start 157.5125 79.11375) (end 157.5125 78.06375) (width 0.5) (layer "B.Cu") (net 3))
 (segment (start 162.0625 79.37375) (end 162.0625 73.92375) (width 0.5) (layer "B.Cu") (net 3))
 (segment (start 152.29625 80.38375) (end 156.2425 80.38375) (width 0.5) (layer "B.Cu") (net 3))
 (segment (start 162.0625 73.92375) (end 163.2825 72.70375) (width 0.5) (layer "B.Cu") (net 3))
 (segment (start 134.0625 84.28375) (end 134.0625 73.172724) (width 0.5) (layer "B.Cu") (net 3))
 (segment (start 134.0725 72.55375) (end 135.2225 71.40375) (width 0.5) (layer "B.Cu") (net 3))
 (segment (start 147.8125 66.59375) (end 150.7325 66.59375) (width 0.5) (layer "B.Cu") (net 3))
 (segment (start 156.2425 80.38375) (end 157.5125 79.11375) (width 0.5) (layer "B.Cu") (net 3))
 (segment (start 158.6025 80.20375) (end 157.5125 79.11375) (width 0.5) (layer "B.Cu") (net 3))
 (segment (start 134.0625 84.28375) (end 136.60625 81.74) (width 1) (layer "B.Cu") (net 3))
 (segment (start 150.7325 69.14) (end 150.7075 69.165) (width 1) (layer "B.Cu") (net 3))
 (segment (start 150.7325 66.59375) (end 150.7325 69.14) (width 1) (layer "B.Cu") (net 3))
 (segment (start 150.94 81.74) (end 152.29625 80.38375) (width 0.5) (layer "B.Cu") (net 3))
 (segment (start 164.6025 81.55375) (end 162.5825 81.55375) (width 0.5) (layer "B.Cu") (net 3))
 (segment (start 163.2825 72.70375) (end 164.6725 72.70375) (width 0.5) (layer "B.Cu") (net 3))
 (segment (start 152.6325 85.41) (end 152.6225 85.4) (width 1) (layer "B.Cu") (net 14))
 (segment (start 154.2175 85.41) (end 152.6325 85.41) (width 1) (layer "B.Cu") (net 14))
 (segment (start 153.48 89.36) (end 153.48 86.1475) (width 1) (layer "B.Cu") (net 14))
 (segment (start 153.48 86.1475) (end 154.2175 85.41) (width 1) (layer "B.Cu") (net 14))
 (segment (start 152.452396 84.10375) (end 155.2725 84.10375) (width 0.5) (layer "B.Cu") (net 12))
 (segment (start 150.7975 85.4) (end 151.156146 85.4) (width 0.5) (layer "B.Cu") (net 12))
 (segment (start 151.156146 85.4) (end 152.452396 84.10375) (width 0.5) (layer "B.Cu") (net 12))
 (segment (start 156.02 83.35625) (end 156.02 81.74) (width 0.5) (layer "B.Cu") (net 12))
 (segment (start 156.02 81.74) (end 158.56 81.74) (width 1) (layer "B.Cu") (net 12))
 (segment (start 155.2725 84.10375) (end 156.02 83.35625) (width 0.5) (layer "B.Cu") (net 12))
 (segment (start 156.02 89.36) (end 156.02 85.4325) (width 1) (layer "B.Cu") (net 15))
 (segment (start 164.6025 84.09375) (end 157.35875 84.09375) (width 1) (layer "B.Cu") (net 15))
 (segment (start 156.02 85.4325) (end 156.0425 85.41) (width 1) (layer "B.Cu") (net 15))
 (segment (start 157.35875 84.09375) (end 156.0425 85.41) (width 1) (layer "B.Cu") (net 15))
 (segment (start 145.9825 73.95375) (end 149.2525 77.22375) (width 1) (layer "B.Cu") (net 16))
 (segment (start 145.9825 71.04375) (end 145.9825 73.95375) (width 1) (layer "B.Cu") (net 16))
 (segment (start 149.2525 77.22375) (end 149.2925 77.18375) (width 1) (layer "B.Cu") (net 16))
 (segment (start 149.2925 77.18375) (end 150.5975 77.18375) (width 1) (layer "B.Cu") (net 16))
 (segment (start 153.265 74.20625) (end 153.2725 74.21375) (width 1) (layer "B.Cu") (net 4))
 (segment (start 153.265 70.76375) (end 153.265 74.20625) (width 1) (layer "B.Cu") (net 4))
 (segment (start 153.2475 74.23875) (end 153.2725 74.21375) (width 1) (layer "B.Cu") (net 4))
 (segment (start 153.2725 77.04875) (end 153.1375 77.18375) (width 1) (layer "B.Cu") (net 4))
 (segment (start 153.2725 74.21375) (end 153.2725 77.04875) (width 1) (layer "B.Cu") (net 4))
 (segment (start 164.6125 91.95375) (end 164.6025 91.94375) (width 1) (layer "B.Cu") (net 11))
 (segment (start 164.6025 91.94375) (end 164.6025 89.17375) (width 1) (layer "B.Cu") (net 11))
 (segment (start 164.6125 92.80375) (end 164.6125 91.95375) (width 1) (layer "B.Cu") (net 11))
 (segment (start 163.3525 94.06375) (end 164.6125 92.80375) (width 1) (layer "B.Cu") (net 11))
 (segment (start 163.3525 101.68375) (end 166.6125 101.68375) (width 1) (layer "B.Cu") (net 10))
 (segment (start 154.6025 67.92375) (end 153.2725 66.59375) (width 0.5) (layer "B.Cu") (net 2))
 (segment (start 164.6725 73.97375) (end 166.0775 73.97375) (width 1) (layer "B.Cu") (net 2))
 (segment (start 166.1225 71.90375) (end 162.1425 67.92375) (width 0.5) (layer "B.Cu") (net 2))
 (segment (start 168.3925 92.28375) (end 166.6125 94.06375) (width 1) (layer "B.Cu") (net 2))
 (segment (start 168.3925 76.28875) (end 168.3925 92.28375) (width 1) (layer "B.Cu") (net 2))
 (segment (start 166.1225 73.92875) (end 166.1225 71.90375) (width 0.5) (layer "B.Cu") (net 2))
 (segment (start 162.1425 67.92375) (end 154.6025 67.92375) (width 0.5) (layer "B.Cu") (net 2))
 (segment (start 166.0775 73.97375) (end 166.1225 73.92875) (width 0.5) (layer "B.Cu") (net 2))
 (segment (start 166.0775 73.97375) (end 168.3925 76.28875) (width 1) (layer "B.Cu") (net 2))
 (segment (start 160.9025 87.38375) (end 161.1225 87.60375) (width 1) (layer "F.Cu") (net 6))
 (segment (start 160.9025 72.32375) (end 160.9025 87.38375) (width 1) (layer "F.Cu") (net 6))
 (segment (start 160.06 78.07125) (end 160.0525 78.06375) (width 1) (layer "F.Cu") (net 6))
 (via (at 160.9025 72.32375) (size 1.75) (drill 1) (layers "F.Cu" "B.Cu") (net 6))
 (via (at 161.1225 87.60375) (size 1.75) (drill 1) (layers "F.Cu" "B.Cu") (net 6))
 (segment (start 159.36625 89.36) (end 161.1225 87.60375) (width 1) (layer "B.Cu") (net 6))
 (segment (start 160.0525 75.91375) (end 158.3525 74.21375) (width 1) (layer "B.Cu") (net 6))
 (segment (start 160.1425 78.17875) (end 160.1475 78.18375) (width 1) (layer "B.Cu") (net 6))
 (segment (start 160.0525 78.06375) (end 160.0525 75.91375) (width 1) (layer "B.Cu") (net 6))
 (segment (start 158.3525 74.21375) (end 159.0125 74.21375) (width 1) (layer "B.Cu") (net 6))
 (segment (start 158.56 89.36) (end 159.36625 89.36) (width 1) (layer "B.Cu") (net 6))
 (segment (start 159.0125 74.21375) (end 160.9025 72.32375) (width 1) (layer "B.Cu") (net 6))
 (segment (start 150.7325 71.67375) (end 155.8125 66.59375) (width 0.5) (layer "F.Cu") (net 1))
 (segment (start 150.7325 74.21375) (end 150.7325 71.67375) (width 0.5) (layer "F.Cu") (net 1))
 (via (at 161.3425 66.59375) (size 1.75) (drill 1) (layers "F.Cu" "B.Cu") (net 1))
 (segment (start 158.3525 66.59375) (end 161.3425 66.59375) (width 1) (layer "B.Cu") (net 1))
 (segment (start 155.8125 66.59375) (end 158.3525 66.59375) (width 1) (layer "B.Cu") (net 1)))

